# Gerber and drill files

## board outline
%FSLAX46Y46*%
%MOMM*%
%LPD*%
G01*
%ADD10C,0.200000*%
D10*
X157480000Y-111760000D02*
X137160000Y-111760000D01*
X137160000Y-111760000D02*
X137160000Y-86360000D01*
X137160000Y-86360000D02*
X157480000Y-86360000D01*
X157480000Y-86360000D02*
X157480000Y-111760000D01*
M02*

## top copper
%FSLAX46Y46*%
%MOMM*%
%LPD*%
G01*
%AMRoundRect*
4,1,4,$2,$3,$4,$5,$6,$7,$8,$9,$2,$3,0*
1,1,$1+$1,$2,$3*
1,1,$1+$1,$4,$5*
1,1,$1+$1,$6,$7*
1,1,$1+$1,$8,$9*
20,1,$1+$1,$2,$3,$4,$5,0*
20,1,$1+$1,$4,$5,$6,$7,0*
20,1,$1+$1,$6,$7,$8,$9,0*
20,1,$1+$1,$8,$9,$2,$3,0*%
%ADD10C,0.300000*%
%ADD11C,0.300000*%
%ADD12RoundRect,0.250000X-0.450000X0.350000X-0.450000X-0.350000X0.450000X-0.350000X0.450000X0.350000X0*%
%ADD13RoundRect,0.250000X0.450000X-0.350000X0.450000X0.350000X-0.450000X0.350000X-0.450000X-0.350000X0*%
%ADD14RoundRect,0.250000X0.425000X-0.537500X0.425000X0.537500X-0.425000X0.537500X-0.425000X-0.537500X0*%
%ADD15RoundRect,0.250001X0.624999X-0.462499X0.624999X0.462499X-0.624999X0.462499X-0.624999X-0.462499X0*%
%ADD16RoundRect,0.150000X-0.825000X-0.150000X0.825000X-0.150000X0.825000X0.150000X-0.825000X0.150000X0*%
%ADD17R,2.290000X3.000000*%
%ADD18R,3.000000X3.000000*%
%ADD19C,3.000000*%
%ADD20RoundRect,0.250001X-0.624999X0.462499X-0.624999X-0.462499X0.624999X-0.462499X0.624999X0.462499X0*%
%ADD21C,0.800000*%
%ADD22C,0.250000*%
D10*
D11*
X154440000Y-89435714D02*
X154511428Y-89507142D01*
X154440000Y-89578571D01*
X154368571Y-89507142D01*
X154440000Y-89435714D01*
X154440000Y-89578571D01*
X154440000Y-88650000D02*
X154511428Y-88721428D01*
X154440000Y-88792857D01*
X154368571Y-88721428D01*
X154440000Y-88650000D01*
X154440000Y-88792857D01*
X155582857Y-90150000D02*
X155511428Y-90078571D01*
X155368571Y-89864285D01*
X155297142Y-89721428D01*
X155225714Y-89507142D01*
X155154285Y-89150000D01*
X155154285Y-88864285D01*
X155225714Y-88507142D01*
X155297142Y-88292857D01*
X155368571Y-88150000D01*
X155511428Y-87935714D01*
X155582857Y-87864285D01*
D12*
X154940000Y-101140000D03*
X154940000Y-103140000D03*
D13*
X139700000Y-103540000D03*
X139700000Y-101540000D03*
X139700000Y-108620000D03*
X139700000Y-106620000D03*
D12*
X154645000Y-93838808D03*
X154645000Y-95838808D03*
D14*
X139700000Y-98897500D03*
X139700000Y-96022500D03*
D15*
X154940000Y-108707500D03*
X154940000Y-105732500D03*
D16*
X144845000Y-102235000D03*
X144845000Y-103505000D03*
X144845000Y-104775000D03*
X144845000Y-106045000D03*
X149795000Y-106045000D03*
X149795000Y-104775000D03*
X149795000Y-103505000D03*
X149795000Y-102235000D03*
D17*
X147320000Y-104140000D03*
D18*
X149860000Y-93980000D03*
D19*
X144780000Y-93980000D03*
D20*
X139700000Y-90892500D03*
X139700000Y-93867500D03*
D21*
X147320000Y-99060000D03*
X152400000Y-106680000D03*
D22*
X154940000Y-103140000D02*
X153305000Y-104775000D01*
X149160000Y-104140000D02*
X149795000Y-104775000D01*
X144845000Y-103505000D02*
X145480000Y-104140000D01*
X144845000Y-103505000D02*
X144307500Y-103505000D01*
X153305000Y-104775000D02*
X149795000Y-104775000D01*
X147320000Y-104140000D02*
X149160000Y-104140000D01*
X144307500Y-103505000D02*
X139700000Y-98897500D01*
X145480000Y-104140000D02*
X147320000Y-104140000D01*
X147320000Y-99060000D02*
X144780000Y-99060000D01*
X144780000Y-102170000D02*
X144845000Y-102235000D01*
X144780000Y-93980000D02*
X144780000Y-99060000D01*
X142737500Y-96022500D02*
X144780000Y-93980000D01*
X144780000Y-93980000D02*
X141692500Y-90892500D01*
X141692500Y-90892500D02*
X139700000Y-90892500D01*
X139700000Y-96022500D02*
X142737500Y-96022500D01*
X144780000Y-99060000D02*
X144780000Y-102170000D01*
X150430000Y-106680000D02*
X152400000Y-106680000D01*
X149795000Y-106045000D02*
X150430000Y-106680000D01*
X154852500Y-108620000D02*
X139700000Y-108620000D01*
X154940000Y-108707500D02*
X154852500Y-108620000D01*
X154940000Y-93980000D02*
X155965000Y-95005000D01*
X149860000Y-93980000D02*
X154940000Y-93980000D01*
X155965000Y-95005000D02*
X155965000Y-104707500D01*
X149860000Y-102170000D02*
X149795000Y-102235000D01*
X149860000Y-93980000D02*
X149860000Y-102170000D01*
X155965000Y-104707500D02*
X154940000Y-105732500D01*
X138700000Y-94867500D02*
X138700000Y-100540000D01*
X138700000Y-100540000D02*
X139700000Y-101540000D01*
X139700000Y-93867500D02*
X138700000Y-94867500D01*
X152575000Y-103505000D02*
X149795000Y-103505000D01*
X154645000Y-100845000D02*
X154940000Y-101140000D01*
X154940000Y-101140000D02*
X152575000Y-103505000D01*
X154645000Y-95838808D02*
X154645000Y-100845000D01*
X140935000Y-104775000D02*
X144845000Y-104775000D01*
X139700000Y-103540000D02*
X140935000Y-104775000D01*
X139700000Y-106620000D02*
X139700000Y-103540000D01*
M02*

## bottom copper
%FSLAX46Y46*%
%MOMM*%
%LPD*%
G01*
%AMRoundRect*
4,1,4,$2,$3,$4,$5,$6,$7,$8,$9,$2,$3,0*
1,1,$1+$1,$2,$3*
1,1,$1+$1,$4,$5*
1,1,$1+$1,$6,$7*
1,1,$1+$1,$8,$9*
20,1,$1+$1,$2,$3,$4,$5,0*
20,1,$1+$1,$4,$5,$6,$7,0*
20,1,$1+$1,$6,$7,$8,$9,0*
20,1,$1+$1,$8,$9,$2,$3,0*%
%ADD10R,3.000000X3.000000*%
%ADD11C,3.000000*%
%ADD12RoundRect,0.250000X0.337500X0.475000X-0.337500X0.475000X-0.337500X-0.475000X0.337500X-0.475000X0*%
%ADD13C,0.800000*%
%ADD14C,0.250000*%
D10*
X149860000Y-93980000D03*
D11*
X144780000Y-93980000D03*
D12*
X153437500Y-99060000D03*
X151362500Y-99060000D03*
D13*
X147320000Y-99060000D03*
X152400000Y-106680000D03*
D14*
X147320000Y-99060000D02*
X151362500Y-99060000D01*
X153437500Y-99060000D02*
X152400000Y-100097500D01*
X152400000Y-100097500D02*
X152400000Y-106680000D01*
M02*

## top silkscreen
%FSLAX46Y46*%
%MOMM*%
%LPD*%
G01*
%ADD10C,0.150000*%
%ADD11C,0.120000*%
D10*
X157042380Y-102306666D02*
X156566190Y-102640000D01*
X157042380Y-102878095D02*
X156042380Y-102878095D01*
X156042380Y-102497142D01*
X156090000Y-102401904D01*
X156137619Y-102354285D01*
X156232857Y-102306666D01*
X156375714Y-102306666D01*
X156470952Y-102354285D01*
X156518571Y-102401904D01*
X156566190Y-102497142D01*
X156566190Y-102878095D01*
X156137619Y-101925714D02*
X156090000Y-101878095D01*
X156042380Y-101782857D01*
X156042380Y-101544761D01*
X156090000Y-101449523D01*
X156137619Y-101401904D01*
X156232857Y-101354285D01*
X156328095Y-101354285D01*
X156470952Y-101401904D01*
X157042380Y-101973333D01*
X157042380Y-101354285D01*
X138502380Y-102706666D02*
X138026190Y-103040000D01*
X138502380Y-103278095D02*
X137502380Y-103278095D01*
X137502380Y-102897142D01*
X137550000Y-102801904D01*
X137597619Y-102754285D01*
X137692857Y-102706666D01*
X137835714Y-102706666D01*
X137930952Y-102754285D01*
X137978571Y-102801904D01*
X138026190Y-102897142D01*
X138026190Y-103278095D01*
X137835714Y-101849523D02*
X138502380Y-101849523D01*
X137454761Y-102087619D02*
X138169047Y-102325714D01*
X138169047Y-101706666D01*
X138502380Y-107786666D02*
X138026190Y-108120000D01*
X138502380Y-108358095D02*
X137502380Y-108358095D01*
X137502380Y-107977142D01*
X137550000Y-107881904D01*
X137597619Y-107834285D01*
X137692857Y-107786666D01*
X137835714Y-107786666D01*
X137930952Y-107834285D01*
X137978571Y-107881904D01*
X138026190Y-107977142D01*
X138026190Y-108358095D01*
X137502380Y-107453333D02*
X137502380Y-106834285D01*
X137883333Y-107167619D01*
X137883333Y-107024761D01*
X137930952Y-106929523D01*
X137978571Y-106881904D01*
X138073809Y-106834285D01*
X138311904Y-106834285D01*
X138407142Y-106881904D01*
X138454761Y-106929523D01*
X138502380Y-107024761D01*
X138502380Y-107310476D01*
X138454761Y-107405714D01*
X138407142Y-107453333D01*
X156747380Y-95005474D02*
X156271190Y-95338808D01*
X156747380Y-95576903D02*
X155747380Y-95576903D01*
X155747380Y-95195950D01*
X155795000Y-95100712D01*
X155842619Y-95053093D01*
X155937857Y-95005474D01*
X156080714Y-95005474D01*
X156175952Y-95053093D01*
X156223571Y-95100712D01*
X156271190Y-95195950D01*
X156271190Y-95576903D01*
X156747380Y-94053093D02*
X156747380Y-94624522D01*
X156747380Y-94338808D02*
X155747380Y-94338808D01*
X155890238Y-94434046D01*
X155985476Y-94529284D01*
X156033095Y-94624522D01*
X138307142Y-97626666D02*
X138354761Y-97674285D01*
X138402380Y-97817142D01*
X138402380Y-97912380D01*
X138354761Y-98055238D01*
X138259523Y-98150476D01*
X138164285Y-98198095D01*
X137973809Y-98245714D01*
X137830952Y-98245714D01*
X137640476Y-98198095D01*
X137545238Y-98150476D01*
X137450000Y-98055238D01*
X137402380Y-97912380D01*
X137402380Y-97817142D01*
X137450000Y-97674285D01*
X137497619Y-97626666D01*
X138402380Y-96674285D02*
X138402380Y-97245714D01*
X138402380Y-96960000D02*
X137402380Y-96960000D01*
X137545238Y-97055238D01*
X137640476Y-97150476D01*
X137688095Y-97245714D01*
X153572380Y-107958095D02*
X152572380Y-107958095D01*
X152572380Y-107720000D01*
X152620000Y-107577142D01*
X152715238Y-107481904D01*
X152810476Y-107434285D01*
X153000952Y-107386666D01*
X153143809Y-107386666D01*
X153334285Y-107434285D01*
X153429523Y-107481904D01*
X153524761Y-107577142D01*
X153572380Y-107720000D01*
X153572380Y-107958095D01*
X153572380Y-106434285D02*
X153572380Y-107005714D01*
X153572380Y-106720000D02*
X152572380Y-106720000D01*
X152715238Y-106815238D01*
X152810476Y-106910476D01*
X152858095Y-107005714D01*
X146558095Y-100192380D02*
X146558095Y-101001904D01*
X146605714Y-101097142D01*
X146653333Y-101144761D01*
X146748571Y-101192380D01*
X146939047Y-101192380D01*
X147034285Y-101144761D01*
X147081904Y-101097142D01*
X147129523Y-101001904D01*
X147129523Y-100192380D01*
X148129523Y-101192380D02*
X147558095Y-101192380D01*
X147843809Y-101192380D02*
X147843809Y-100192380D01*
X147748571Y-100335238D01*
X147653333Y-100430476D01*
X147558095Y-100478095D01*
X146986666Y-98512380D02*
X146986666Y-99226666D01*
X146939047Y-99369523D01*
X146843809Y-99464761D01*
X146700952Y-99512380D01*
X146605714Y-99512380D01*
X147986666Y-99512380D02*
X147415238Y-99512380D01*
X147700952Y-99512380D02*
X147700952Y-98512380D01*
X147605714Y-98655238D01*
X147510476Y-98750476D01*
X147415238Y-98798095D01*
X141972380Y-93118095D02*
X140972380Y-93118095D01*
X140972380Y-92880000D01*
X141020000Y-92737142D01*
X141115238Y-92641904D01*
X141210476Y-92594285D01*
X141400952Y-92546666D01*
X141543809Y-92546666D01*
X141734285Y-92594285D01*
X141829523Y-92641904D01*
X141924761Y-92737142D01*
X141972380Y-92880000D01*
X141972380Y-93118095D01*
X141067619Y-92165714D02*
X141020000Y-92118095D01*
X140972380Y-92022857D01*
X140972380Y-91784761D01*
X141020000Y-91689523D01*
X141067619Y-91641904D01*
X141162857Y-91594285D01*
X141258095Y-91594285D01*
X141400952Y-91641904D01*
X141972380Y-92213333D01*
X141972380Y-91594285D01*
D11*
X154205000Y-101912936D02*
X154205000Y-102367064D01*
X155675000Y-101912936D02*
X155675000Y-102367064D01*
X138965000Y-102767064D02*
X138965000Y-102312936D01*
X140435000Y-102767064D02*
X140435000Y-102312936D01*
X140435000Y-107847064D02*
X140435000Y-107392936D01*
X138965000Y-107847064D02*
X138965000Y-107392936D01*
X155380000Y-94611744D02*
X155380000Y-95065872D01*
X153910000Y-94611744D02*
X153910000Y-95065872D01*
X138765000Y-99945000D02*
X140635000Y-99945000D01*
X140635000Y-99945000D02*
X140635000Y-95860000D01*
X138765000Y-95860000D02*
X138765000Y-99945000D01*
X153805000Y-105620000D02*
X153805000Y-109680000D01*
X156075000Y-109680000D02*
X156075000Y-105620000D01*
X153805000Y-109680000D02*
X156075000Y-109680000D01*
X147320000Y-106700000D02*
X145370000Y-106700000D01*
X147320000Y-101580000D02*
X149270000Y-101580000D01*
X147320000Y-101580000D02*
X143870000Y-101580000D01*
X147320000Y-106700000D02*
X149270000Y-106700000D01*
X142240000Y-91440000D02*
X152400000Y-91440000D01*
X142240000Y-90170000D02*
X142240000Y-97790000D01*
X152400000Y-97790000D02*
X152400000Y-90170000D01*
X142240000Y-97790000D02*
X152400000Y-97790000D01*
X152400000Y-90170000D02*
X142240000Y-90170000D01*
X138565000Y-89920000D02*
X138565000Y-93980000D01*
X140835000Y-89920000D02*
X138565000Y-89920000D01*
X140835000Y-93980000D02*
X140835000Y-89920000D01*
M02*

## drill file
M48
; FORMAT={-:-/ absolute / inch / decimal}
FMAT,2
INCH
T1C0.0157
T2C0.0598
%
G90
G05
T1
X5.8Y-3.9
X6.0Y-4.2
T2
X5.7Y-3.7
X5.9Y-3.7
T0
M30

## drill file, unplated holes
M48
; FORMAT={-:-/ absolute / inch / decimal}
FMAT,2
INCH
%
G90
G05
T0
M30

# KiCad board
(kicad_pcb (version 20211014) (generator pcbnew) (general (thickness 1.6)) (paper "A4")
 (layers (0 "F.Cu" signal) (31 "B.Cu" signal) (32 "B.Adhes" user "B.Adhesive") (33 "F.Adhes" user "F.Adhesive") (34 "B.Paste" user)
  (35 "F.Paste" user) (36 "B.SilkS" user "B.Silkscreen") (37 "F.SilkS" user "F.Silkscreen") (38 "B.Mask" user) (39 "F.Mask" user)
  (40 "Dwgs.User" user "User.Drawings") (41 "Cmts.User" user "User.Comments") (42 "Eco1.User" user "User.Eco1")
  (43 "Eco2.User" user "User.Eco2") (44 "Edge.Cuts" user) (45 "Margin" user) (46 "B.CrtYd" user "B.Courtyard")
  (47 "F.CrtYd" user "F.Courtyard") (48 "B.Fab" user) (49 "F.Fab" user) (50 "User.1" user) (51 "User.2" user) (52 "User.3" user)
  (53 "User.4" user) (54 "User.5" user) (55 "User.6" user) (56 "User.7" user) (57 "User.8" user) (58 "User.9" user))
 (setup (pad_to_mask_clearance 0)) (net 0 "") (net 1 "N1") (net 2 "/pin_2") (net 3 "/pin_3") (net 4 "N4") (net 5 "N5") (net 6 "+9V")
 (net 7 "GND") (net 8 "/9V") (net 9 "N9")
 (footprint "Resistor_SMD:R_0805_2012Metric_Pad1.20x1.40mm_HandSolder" (layer "F.Cu") (at 154.94 102.14 -90)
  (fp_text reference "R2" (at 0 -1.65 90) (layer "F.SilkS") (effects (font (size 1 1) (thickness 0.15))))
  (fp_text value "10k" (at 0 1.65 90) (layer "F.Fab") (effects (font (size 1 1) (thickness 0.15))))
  (fp_line (start -0.227064 0.735) (end 0.227064 0.735) (layer "F.SilkS") (width 0.12))
  (fp_line (start -0.227064 -0.735) (end 0.227064 -0.735) (layer "F.SilkS") (width 0.12))
  (pad "1" smd roundrect (at -1 0 270) (size 1.2 1.4) (layers "F.Cu" "F.Paste" "F.Mask") (roundrect_rratio 0.2083333333) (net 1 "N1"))
  (pad "2" smd roundrect (at 1 0 270) (size 1.2 1.4) (layers "F.Cu" "F.Paste" "F.Mask") (roundrect_rratio 0.2083333333) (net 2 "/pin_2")))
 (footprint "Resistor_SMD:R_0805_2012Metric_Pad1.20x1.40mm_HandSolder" (layer "F.Cu") (at 139.7 102.54 90)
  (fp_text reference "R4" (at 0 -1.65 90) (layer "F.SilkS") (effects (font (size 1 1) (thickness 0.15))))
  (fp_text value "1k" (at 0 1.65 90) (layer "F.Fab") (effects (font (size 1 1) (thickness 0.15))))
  (fp_line (start -0.227064 -0.735) (end 0.227064 -0.735) (layer "F.SilkS") (width 0.12))
  (fp_line (start -0.227064 0.735) (end 0.227064 0.735) (layer "F.SilkS") (width 0.12))
  (pad "1" smd roundrect (at -1 0 90) (size 1.2 1.4) (layers "F.Cu" "F.Paste" "F.Mask") (roundrect_rratio 0.2083333333) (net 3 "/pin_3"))
  (pad "2" smd roundrect (at 1 0 90) (size 1.2 1.4) (layers "F.Cu" "F.Paste" "F.Mask") (roundrect_rratio 0.2083333333) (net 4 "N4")))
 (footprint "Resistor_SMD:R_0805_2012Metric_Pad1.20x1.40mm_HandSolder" (layer "F.Cu") (at 139.7 107.62 90)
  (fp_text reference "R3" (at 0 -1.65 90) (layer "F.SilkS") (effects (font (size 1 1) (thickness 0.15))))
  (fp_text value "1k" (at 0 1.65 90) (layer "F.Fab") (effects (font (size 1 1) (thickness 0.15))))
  (fp_line (start -0.227064 0.735) (end 0.227064 0.735) (layer "F.SilkS") (width 0.12))
  (fp_line (start -0.227064 -0.735) (end 0.227064 -0.735) (layer "F.SilkS") (width 0.12))
  (pad "1" smd roundrect (at -1 0 90) (size 1.2 1.4) (layers "F.Cu" "F.Paste" "F.Mask") (roundrect_rratio 0.2083333333) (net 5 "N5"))
  (pad "2" smd roundrect (at 1 0 90) (size 1.2 1.4) (layers "F.Cu" "F.Paste" "F.Mask") (roundrect_rratio 0.2083333333) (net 3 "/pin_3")))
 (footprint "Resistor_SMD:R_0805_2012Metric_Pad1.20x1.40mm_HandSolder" (layer "F.Cu") (at 154.645 94.838808 -90)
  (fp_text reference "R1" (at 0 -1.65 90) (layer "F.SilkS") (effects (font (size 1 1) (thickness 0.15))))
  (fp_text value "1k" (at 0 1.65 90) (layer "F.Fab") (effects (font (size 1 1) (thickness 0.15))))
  (fp_line (start -0.227064 -0.735) (end 0.227064 -0.735) (layer "F.SilkS") (width 0.12))
  (fp_line (start -0.227064 0.735) (end 0.227064 0.735) (layer "F.SilkS") (width 0.12))
  (pad "1" smd roundrect (at -1 0 270) (size 1.2 1.4) (layers "F.Cu" "F.Paste" "F.Mask") (roundrect_rratio 0.2083333333) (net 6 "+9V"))
  (pad "2" smd roundrect (at 1 0 270) (size 1.2 1.4) (layers "F.Cu" "F.Paste" "F.Mask") (roundrect_rratio 0.2083333333) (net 1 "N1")))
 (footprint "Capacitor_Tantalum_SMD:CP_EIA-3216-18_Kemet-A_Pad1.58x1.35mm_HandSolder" (layer "F.Cu") (at 139.7 97.46 90)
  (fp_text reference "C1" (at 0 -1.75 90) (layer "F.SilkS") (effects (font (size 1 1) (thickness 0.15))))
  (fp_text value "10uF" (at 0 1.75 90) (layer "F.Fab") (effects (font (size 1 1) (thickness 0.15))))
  (fp_line (start -2.485 -0.935) (end -2.485 0.935) (layer "F.SilkS") (width 0.12))
  (fp_line (start -2.485 0.935) (end 1.6 0.935) (layer "F.SilkS") (width 0.12))
  (fp_line (start 1.6 -0.935) (end -2.485 -0.935) (layer "F.SilkS") (width 0.12))
  (pad "1" smd roundrect (at -1.4375 0 90) (size 1.575 1.35) (layers "F.Cu" "F.Paste" "F.Mask") (roundrect_rratio 0.1851851852)
   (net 2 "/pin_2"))
  (pad "2" smd roundrect (at 1.4375 0 90) (size 1.575 1.35) (layers "F.Cu" "F.Paste" "F.Mask") (roundrect_rratio 0.1851851852) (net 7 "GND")))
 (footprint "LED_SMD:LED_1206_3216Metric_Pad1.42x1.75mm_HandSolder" (layer "F.Cu") (at 154.94 107.22 90)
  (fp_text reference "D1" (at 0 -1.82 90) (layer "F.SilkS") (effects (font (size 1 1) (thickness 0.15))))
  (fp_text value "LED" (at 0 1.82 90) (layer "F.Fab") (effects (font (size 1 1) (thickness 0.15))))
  (fp_line (start 1.6 -1.135) (end -2.46 -1.135) (layer "F.SilkS") (width 0.12))
  (fp_line (start -2.46 1.135) (end 1.6 1.135) (layer "F.SilkS") (width 0.12))
  (fp_line (start -2.46 -1.135) (end -2.46 1.135) (layer "F.SilkS") (width 0.12))
  (pad "1" smd roundrect (at -1.4875 0 90) (size 1.425 1.75) (layers "F.Cu" "F.Paste" "F.Mask") (roundrect_rratio 0.1754392982) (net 5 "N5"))
  (pad "2" smd roundrect (at 1.4875 0 90) (size 1.425 1.75) (layers "F.Cu" "F.Paste" "F.Mask") (roundrect_rratio 0.1754392982) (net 6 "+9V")))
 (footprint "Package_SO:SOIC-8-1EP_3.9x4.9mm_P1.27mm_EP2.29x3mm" (layer "F.Cu") (at 147.32 104.14)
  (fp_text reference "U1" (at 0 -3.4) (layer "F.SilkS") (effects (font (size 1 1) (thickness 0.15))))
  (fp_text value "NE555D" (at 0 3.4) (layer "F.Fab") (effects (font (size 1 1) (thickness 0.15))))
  (fp_line (start 0 2.56) (end -1.95 2.56) (layer "F.SilkS") (width 0.12))
  (fp_line (start 0 -2.56) (end 1.95 -2.56) (layer "F.SilkS") (width 0.12))
  (fp_line (start 0 -2.56) (end -3.45 -2.56) (layer "F.SilkS") (width 0.12))
  (fp_line (start 0 2.56) (end 1.95 2.56) (layer "F.SilkS") (width 0.12))
  (pad "" smd roundrect (at -0.57 0.75) (size 0.92 1.21) (layers "F.Paste") (roundrect_rratio 0.25))
  (pad "" smd roundrect (at -0.57 -0.75) (size 0.92 1.21) (layers "F.Paste") (roundrect_rratio 0.25))
  (pad "" smd roundrect (at 0.57 -0.75) (size 0.92 1.21) (layers "F.Paste") (roundrect_rratio 0.25))
  (pad "" smd roundrect (at 0.57 0.75) (size 0.92 1.21) (layers "F.Paste") (roundrect_rratio 0.25))
  (pad "1" smd roundrect (at -2.475 -1.905) (size 1.95 0.6) (layers "F.Cu" "F.Paste" "F.Mask") (roundrect_rratio 0.25) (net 7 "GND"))
  (pad "2" smd roundrect (at -2.475 -0.635) (size 1.95 0.6) (layers "F.Cu" "F.Paste" "F.Mask") (roundrect_rratio 0.25) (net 2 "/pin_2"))
  (pad "3" smd roundrect (at -2.475 0.635) (size 1.95 0.6) (layers "F.Cu" "F.Paste" "F.Mask") (roundrect_rratio 0.25) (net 3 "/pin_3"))
  (pad "4" smd roundrect (at -2.475 1.905) (size 1.95 0.6) (layers "F.Cu" "F.Paste" "F.Mask") (roundrect_rratio 0.25) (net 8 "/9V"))
  (pad "5" smd roundrect (at 2.475 1.905) (size 1.95 0.6) (layers "F.Cu" "F.Paste" "F.Mask") (roundrect_rratio 0.25) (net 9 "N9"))
  (pad "6" smd roundrect (at 2.475 0.635) (size 1.95 0.6) (layers "F.Cu" "F.Paste" "F.Mask") (roundrect_rratio 0.25) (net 2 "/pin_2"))
  (pad "7" smd roundrect (at 2.475 -0.635) (size 1.95 0.6) (layers "F.Cu" "F.Paste" "F.Mask") (roundrect_rratio 0.25) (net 1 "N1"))
  (pad "8" smd roundrect (at 2.475 -1.905) (size 1.95 0.6) (layers "F.Cu" "F.Paste" "F.Mask") (roundrect_rratio 0.25) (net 6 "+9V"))
  (pad "9" smd rect (at 0 0) (size 2.29 3) (layers "F.Cu" "F.Mask") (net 2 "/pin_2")))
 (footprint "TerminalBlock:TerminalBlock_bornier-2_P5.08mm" (layer "F.Cu") (at 149.86 93.98 180)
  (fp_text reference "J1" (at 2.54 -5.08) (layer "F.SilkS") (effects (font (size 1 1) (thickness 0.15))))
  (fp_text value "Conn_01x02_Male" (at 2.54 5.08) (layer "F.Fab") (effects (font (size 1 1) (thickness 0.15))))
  (fp_line (start 7.62 2.54) (end -2.54 2.54) (layer "F.SilkS") (width 0.12))
  (fp_line (start 7.62 3.81) (end 7.62 -3.81) (layer "F.SilkS") (width 0.12))
  (fp_line (start -2.54 -3.81) (end -2.54 3.81) (layer "F.SilkS") (width 0.12))
  (fp_line (start 7.62 -3.81) (end -2.54 -3.81) (layer "F.SilkS") (width 0.12))
  (fp_line (start -2.54 3.81) (end 7.62 3.81) (layer "F.SilkS") (width 0.12))
  (pad "1" thru_hole rect (at 0 0 180) (size 3 3) (drill 1.52) (layers *.Cu *.Mask) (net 6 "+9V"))
  (pad "2" thru_hole circle (at 5.08 0 180) (size 3 3) (drill 1.52) (layers *.Cu *.Mask) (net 7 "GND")))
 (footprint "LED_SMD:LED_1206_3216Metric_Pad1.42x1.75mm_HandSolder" (layer "F.Cu") (at 139.7 92.38 -90)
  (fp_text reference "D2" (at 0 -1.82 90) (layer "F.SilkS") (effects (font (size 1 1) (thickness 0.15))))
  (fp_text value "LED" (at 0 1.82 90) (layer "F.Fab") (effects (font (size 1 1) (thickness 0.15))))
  (fp_line (start -2.46 1.135) (end 1.6 1.135) (layer "F.SilkS") (width 0.12))
  (fp_line (start -2.46 -1.135) (end -2.46 1.135) (layer "F.SilkS") (width 0.12))
  (fp_line (start 1.6 -1.135) (end -2.46 -1.135) (layer "F.SilkS") (width 0.12))
  (pad "1" smd roundrect (at -1.4875 0 270) (size 1.425 1.75) (layers "F.Cu" "F.Paste" "F.Mask") (roundrect_rratio 0.1754392982)
   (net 7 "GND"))
  (pad "2" smd roundrect (at 1.4875 0 270) (size 1.425 1.75) (layers "F.Cu" "F.Paste" "F.Mask") (roundrect_rratio 0.1754392982) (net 4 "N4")))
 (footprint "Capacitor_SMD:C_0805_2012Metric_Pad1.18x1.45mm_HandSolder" (layer "B.Cu") (at 152.4 99.06 180)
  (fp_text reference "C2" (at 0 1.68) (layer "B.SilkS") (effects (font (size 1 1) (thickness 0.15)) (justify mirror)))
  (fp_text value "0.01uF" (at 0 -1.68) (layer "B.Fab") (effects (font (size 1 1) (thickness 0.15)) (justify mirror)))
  (pad "1" smd roundrect (at -1.0375 0 180) (size 1.175 1.45) (layers "B.Cu" "B.Paste" "B.Mask") (roundrect_rratio 0.2127659574)
   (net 9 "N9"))
  (pad "2" smd roundrect (at 1.0375 0 180) (size 1.175 1.45) (layers "B.Cu" "B.Paste" "B.Mask") (roundrect_rratio 0.2127659574)
   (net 7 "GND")))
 (gr_rect (start 157.48 111.76) (end 137.16 86.36) (layer "Edge.Cuts") (width 0.2) (fill none))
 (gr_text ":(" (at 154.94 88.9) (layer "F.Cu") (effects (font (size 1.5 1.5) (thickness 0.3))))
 (segment (start 154.94 103.14) (end 153.305 104.775) (width 0.25) (layer "F.Cu") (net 2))
 (segment (start 149.16 104.14) (end 149.795 104.775) (width 0.25) (layer "F.Cu") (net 2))
 (segment (start 144.845 103.505) (end 145.48 104.14) (width 0.25) (layer "F.Cu") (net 2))
 (segment (start 144.845 103.505) (end 144.3075 103.505) (width 0.25) (layer "F.Cu") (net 2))
 (segment (start 153.305 104.775) (end 149.795 104.775) (width 0.25) (layer "F.Cu") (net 2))
 (segment (start 147.32 104.14) (end 149.16 104.14) (width 0.25) (layer "F.Cu") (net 2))
 (segment (start 144.3075 103.505) (end 139.7 98.8975) (width 0.25) (layer "F.Cu") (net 2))
 (segment (start 145.48 104.14) (end 147.32 104.14) (width 0.25) (layer "F.Cu") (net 2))
 (segment (start 147.32 99.06) (end 144.78 99.06) (width 0.25) (layer "F.Cu") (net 7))
 (segment (start 144.78 102.17) (end 144.845 102.235) (width 0.25) (layer "F.Cu") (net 7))
 (segment (start 144.78 93.98) (end 144.78 99.06) (width 0.25) (layer "F.Cu") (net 7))
 (segment (start 142.7375 96.0225) (end 144.78 93.98) (width 0.25) (layer "F.Cu") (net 7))
 (segment (start 144.78 93.98) (end 141.6925 90.8925) (width 0.25) (layer "F.Cu") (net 7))
 (segment (start 141.6925 90.8925) (end 139.7 90.8925) (width 0.25) (layer "F.Cu") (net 7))
 (segment (start 139.7 96.0225) (end 142.7375 96.0225) (width 0.25) (layer "F.Cu") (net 7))
 (segment (start 144.78 99.06) (end 144.78 102.17) (width 0.25) (layer "F.Cu") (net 7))
 (via (at 147.32 99.06) (size 0.8) (drill 0.4) (layers "F.Cu" "B.Cu") (free) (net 7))
 (segment (start 147.32 99.06) (end 151.3625 99.06) (width 0.25) (layer "B.Cu") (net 7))
 (segment (start 150.43 106.68) (end 152.4 106.68) (width 0.25) (layer "F.Cu") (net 9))
 (segment (start 149.795 106.045) (end 150.43 106.68) (width 0.25) (layer "F.Cu") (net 9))
 (via (at 152.4 106.68) (size 0.8) (drill 0.4) (layers "F.Cu" "B.Cu") (free) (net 9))
 (segment (start 153.4375 99.06) (end 152.4 100.0975) (width 0.25) (layer "B.Cu") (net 9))
 (segment (start 152.4 100.0975) (end 152.4 106.68) (width 0.25) (layer "B.Cu") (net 9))
 (segment (start 154.8525 108.62) (end 139.7 108.62) (width 0.25) (layer "F.Cu") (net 5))
 (segment (start 154.94 108.7075) (end 154.8525 108.62) (width 0.25) (layer "F.Cu") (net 5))
 (segment (start 154.94 93.98) (end 155.965 95.005) (width 0.25) (layer "F.Cu") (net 6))
 (segment (start 149.86 93.98) (end 154.94 93.98) (width 0.25) (layer "F.Cu") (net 6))
 (segment (start 155.965 95.005) (end 155.965 104.7075) (width 0.25) (layer "F.Cu") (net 6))
 (segment (start 149.86 102.17) (end 149.795 102.235) (width 0.25) (layer "F.Cu") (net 6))
 (segment (start 149.86 93.98) (end 149.86 102.17) (width 0.25) (layer "F.Cu") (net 6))
 (segment (start 155.965 104.7075) (end 154.94 105.7325) (width 0.25) (layer "F.Cu") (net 6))
 (segment (start 138.7 94.8675) (end 138.7 100.54) (width 0.25) (layer "F.Cu") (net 4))
 (segment (start 138.7 100.54) (end 139.7 101.54) (width 0.25) (layer "F.Cu") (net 4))
 (segment (start 139.7 93.8675) (end 138.7 94.8675) (width 0.25) (layer "F.Cu") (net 4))
 (segment (start 152.575 103.505) (end 149.795 103.505) (width 0.25) (layer "F.Cu") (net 1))
 (segment (start 154.645 100.845) (end 154.94 101.14) (width 0.25) (layer "F.Cu") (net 1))
 (segment (start 154.94 101.14) (end 152.575 103.505) (width 0.25) (layer "F.Cu") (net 1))
 (segment (start 154.645 95.838808) (end 154.645 100.845) (width 0.25) (layer "F.Cu") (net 1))
 (segment (start 140.935 104.775) (end 144.845 104.775) (width 0.25) (layer "F.Cu") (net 3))
 (segment (start 139.7 103.54) (end 140.935 104.775) (width 0.25) (layer "F.Cu") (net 3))
 (segment (start 139.7 106.62) (end 139.7 103.54) (width 0.25) (layer "F.Cu") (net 3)))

